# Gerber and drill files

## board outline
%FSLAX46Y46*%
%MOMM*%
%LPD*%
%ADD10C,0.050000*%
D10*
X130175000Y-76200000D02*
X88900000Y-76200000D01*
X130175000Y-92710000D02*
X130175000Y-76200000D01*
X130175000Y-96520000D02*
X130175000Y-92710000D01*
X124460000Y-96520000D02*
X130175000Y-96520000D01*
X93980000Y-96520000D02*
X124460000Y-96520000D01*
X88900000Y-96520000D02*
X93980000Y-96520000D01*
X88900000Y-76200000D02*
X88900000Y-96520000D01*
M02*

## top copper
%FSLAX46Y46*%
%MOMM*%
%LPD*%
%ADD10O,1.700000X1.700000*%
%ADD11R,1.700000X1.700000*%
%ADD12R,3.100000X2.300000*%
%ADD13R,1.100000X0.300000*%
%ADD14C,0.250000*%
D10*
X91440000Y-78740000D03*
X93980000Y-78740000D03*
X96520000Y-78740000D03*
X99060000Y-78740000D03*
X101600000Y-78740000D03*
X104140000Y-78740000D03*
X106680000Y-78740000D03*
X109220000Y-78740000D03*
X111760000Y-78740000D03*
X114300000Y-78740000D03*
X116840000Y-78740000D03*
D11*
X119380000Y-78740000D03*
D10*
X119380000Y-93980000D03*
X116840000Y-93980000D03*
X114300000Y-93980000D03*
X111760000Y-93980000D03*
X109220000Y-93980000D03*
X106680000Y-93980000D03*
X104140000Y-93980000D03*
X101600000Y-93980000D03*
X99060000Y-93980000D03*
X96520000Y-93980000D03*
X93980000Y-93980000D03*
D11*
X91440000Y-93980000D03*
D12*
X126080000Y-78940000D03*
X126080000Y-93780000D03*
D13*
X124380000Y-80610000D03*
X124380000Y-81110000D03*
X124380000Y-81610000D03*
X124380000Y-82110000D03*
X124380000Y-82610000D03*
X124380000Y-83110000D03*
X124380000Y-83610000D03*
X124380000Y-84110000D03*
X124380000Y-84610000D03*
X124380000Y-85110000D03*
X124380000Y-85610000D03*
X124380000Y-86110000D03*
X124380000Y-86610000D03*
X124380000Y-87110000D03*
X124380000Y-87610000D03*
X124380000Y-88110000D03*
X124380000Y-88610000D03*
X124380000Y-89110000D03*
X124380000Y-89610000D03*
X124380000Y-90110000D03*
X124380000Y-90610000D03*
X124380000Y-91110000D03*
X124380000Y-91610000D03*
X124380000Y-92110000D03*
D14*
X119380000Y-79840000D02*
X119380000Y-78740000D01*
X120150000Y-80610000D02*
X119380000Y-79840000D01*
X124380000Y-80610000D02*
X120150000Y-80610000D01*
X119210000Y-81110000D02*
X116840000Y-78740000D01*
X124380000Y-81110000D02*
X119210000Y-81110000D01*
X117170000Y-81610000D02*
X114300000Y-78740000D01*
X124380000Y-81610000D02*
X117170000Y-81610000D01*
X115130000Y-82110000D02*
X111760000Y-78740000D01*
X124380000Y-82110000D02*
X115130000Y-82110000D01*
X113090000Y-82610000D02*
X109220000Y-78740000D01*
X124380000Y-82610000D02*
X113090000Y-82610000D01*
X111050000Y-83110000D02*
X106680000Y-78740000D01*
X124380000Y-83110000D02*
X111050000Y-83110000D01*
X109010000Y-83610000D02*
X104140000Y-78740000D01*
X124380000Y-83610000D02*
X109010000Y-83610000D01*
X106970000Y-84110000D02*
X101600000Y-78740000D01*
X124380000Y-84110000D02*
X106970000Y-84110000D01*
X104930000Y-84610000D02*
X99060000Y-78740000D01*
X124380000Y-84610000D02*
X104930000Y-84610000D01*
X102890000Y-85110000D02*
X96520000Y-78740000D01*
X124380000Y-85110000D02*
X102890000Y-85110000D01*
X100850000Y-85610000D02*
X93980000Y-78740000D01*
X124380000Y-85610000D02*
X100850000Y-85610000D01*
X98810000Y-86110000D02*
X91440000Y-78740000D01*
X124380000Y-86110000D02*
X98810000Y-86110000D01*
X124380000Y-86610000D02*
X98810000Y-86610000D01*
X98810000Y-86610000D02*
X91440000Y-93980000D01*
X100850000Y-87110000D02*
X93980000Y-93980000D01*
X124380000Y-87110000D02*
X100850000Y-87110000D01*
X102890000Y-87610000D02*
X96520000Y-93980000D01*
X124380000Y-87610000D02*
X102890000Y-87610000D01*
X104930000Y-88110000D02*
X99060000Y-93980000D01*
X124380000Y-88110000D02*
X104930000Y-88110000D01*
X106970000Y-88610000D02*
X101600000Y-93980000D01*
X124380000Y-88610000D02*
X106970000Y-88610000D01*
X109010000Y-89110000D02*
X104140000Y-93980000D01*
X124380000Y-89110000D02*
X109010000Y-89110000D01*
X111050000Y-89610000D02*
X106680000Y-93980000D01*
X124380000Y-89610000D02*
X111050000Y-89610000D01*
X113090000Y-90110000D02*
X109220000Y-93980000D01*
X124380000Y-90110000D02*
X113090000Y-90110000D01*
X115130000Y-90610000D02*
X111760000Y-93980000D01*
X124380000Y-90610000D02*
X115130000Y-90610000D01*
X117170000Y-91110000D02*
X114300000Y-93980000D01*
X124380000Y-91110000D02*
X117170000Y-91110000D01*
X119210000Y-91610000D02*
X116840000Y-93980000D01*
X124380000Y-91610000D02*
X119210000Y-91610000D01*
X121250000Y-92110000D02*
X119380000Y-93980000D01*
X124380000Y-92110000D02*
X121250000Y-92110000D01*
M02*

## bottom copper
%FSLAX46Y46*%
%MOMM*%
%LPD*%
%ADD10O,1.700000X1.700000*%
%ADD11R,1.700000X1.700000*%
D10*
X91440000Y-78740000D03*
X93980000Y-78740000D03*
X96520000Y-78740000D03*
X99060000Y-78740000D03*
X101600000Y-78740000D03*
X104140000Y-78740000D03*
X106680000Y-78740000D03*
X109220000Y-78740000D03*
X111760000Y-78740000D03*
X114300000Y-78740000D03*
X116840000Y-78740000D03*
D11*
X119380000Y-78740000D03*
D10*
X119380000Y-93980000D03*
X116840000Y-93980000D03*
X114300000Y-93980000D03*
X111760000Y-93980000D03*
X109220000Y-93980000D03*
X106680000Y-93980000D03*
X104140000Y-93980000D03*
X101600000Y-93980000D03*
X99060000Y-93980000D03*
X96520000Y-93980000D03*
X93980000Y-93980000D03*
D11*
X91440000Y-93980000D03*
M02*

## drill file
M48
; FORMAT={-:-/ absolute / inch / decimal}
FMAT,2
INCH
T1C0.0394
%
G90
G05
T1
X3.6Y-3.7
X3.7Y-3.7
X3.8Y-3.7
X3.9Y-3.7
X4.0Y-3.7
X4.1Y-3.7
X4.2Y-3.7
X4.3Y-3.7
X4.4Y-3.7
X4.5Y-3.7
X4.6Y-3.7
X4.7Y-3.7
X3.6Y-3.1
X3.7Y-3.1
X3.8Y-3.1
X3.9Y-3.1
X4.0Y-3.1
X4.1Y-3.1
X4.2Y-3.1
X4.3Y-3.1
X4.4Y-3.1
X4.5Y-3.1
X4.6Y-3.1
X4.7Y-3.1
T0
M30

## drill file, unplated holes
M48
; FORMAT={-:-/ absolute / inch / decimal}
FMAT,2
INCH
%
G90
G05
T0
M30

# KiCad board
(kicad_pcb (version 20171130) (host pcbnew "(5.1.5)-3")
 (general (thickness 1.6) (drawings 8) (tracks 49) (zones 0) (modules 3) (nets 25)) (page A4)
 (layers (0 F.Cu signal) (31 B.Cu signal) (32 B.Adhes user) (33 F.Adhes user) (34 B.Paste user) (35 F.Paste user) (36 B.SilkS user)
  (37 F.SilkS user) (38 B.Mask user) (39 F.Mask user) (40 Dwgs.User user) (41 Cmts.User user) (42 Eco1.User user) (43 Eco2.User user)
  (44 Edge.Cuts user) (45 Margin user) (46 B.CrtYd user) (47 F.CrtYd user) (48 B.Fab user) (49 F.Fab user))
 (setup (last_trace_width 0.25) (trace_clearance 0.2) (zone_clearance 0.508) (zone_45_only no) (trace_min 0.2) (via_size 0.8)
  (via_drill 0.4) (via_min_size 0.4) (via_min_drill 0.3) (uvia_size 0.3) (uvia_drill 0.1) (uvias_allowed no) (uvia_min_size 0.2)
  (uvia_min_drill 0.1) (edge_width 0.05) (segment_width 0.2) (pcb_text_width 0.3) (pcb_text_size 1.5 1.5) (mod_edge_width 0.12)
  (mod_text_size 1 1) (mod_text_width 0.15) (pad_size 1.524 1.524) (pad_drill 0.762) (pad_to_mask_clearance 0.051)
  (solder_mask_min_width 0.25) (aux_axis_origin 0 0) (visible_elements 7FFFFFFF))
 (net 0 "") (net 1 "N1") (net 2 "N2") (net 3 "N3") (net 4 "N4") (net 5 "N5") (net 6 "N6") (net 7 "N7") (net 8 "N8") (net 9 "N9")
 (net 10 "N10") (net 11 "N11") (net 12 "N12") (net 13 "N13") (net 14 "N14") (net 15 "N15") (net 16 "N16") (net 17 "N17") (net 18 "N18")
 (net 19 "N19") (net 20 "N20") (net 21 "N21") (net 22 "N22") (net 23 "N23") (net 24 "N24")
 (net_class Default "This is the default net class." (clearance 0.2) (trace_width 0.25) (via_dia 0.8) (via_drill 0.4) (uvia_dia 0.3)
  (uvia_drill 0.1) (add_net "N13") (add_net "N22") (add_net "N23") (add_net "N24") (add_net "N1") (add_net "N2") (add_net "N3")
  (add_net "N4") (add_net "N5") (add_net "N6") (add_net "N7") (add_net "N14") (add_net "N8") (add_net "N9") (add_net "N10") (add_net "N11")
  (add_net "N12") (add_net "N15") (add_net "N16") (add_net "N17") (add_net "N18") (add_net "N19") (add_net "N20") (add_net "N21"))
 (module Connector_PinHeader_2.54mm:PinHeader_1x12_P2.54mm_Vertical (layer F.Cu) (at 119.38 78.74 270)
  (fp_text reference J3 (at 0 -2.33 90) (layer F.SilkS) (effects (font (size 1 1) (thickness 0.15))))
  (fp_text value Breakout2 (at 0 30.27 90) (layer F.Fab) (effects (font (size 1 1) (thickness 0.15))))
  (pad 12 thru_hole oval (at 0 27.94 270) (size 1.7 1.7) (drill 1) (layers *.Cu *.Mask) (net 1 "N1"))
  (pad 11 thru_hole oval (at 0 25.4 270) (size 1.7 1.7) (drill 1) (layers *.Cu *.Mask) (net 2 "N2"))
  (pad 10 thru_hole oval (at 0 22.86 270) (size 1.7 1.7) (drill 1) (layers *.Cu *.Mask) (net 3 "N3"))
  (pad 9 thru_hole oval (at 0 20.32 270) (size 1.7 1.7) (drill 1) (layers *.Cu *.Mask) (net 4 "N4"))
  (pad 8 thru_hole oval (at 0 17.78 270) (size 1.7 1.7) (drill 1) (layers *.Cu *.Mask) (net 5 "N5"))
  (pad 7 thru_hole oval (at 0 15.24 270) (size 1.7 1.7) (drill 1) (layers *.Cu *.Mask) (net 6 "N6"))
  (pad 6 thru_hole oval (at 0 12.7 270) (size 1.7 1.7) (drill 1) (layers *.Cu *.Mask) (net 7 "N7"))
  (pad 5 thru_hole oval (at 0 10.16 270) (size 1.7 1.7) (drill 1) (layers *.Cu *.Mask) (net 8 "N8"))
  (pad 4 thru_hole oval (at 0 7.62 270) (size 1.7 1.7) (drill 1) (layers *.Cu *.Mask) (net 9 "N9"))
  (pad 3 thru_hole oval (at 0 5.08 270) (size 1.7 1.7) (drill 1) (layers *.Cu *.Mask) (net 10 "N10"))
  (pad 2 thru_hole oval (at 0 2.54 270) (size 1.7 1.7) (drill 1) (layers *.Cu *.Mask) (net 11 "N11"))
  (pad 1 thru_hole rect (at 0 0 270) (size 1.7 1.7) (drill 1) (layers *.Cu *.Mask) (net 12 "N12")))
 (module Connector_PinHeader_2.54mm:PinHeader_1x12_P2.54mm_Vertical (layer F.Cu) (at 91.44 93.98 90)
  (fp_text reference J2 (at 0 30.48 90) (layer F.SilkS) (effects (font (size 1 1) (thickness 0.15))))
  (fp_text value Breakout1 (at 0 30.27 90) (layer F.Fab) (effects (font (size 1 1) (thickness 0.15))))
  (pad 12 thru_hole oval (at 0 27.94 90) (size 1.7 1.7) (drill 1) (layers *.Cu *.Mask) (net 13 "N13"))
  (pad 11 thru_hole oval (at 0 25.4 90) (size 1.7 1.7) (drill 1) (layers *.Cu *.Mask) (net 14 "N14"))
  (pad 10 thru_hole oval (at 0 22.86 90) (size 1.7 1.7) (drill 1) (layers *.Cu *.Mask) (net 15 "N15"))
  (pad 9 thru_hole oval (at 0 20.32 90) (size 1.7 1.7) (drill 1) (layers *.Cu *.Mask) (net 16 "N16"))
  (pad 8 thru_hole oval (at 0 17.78 90) (size 1.7 1.7) (drill 1) (layers *.Cu *.Mask) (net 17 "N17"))
  (pad 7 thru_hole oval (at 0 15.24 90) (size 1.7 1.7) (drill 1) (layers *.Cu *.Mask) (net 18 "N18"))
  (pad 6 thru_hole oval (at 0 12.7 90) (size 1.7 1.7) (drill 1) (layers *.Cu *.Mask) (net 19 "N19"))
  (pad 5 thru_hole oval (at 0 10.16 90) (size 1.7 1.7) (drill 1) (layers *.Cu *.Mask) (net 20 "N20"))
  (pad 4 thru_hole oval (at 0 7.62 90) (size 1.7 1.7) (drill 1) (layers *.Cu *.Mask) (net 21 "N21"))
  (pad 3 thru_hole oval (at 0 5.08 90) (size 1.7 1.7) (drill 1) (layers *.Cu *.Mask) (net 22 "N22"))
  (pad 2 thru_hole oval (at 0 2.54 90) (size 1.7 1.7) (drill 1) (layers *.Cu *.Mask) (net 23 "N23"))
  (pad 1 thru_hole rect (at 0 0 90) (size 1.7 1.7) (drill 1) (layers *.Cu *.Mask) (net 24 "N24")))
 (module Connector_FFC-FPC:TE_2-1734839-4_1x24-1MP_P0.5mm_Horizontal (layer F.Cu) (at 125.73 86.36 90)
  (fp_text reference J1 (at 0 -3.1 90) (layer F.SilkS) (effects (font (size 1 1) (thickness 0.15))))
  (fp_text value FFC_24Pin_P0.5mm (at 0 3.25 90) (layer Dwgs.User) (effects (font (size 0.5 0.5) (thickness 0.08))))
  (pad MP smd rect (at 7.42 0.35 90) (size 2.3 3.1) (layers F.Cu F.Paste F.Mask))
  (pad MP smd rect (at -7.42 0.35 90) (size 2.3 3.1) (layers F.Cu F.Paste F.Mask))
  (pad 24 smd rect (at 5.75 -1.35 90) (size 0.3 1.1) (layers F.Cu F.Paste F.Mask) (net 12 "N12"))
  (pad 23 smd rect (at 5.25 -1.35 90) (size 0.3 1.1) (layers F.Cu F.Paste F.Mask) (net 11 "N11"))
  (pad 22 smd rect (at 4.75 -1.35 90) (size 0.3 1.1) (layers F.Cu F.Paste F.Mask) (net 10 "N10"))
  (pad 21 smd rect (at 4.25 -1.35 90) (size 0.3 1.1) (layers F.Cu F.Paste F.Mask) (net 9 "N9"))
  (pad 20 smd rect (at 3.75 -1.35 90) (size 0.3 1.1) (layers F.Cu F.Paste F.Mask) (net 8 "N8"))
  (pad 19 smd rect (at 3.25 -1.35 90) (size 0.3 1.1) (layers F.Cu F.Paste F.Mask) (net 7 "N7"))
  (pad 18 smd rect (at 2.75 -1.35 90) (size 0.3 1.1) (layers F.Cu F.Paste F.Mask) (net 6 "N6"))
  (pad 17 smd rect (at 2.25 -1.35 90) (size 0.3 1.1) (layers F.Cu F.Paste F.Mask) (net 5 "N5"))
  (pad 16 smd rect (at 1.75 -1.35 90) (size 0.3 1.1) (layers F.Cu F.Paste F.Mask) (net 4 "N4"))
  (pad 15 smd rect (at 1.25 -1.35 90) (size 0.3 1.1) (layers F.Cu F.Paste F.Mask) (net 3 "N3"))
  (pad 14 smd rect (at 0.75 -1.35 90) (size 0.3 1.1) (layers F.Cu F.Paste F.Mask) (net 2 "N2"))
  (pad 13 smd rect (at 0.25 -1.35 90) (size 0.3 1.1) (layers F.Cu F.Paste F.Mask) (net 1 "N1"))
  (pad 12 smd rect (at -0.25 -1.35 90) (size 0.3 1.1) (layers F.Cu F.Paste F.Mask) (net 24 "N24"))
  (pad 11 smd rect (at -0.75 -1.35 90) (size 0.3 1.1) (layers F.Cu F.Paste F.Mask) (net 23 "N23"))
  (pad 10 smd rect (at -1.25 -1.35 90) (size 0.3 1.1) (layers F.Cu F.Paste F.Mask) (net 22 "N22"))
  (pad 9 smd rect (at -1.75 -1.35 90) (size 0.3 1.1) (layers F.Cu F.Paste F.Mask) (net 21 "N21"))
  (pad 8 smd rect (at -2.25 -1.35 90) (size 0.3 1.1) (layers F.Cu F.Paste F.Mask) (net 20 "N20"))
  (pad 7 smd rect (at -2.75 -1.35 90) (size 0.3 1.1) (layers F.Cu F.Paste F.Mask) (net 19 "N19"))
  (pad 6 smd rect (at -3.25 -1.35 90) (size 0.3 1.1) (layers F.Cu F.Paste F.Mask) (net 18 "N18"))
  (pad 5 smd rect (at -3.75 -1.35 90) (size 0.3 1.1) (layers F.Cu F.Paste F.Mask) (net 17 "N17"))
  (pad 4 smd rect (at -4.25 -1.35 90) (size 0.3 1.1) (layers F.Cu F.Paste F.Mask) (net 16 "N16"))
  (pad 3 smd rect (at -4.75 -1.35 90) (size 0.3 1.1) (layers F.Cu F.Paste F.Mask) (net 15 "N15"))
  (pad 2 smd rect (at -5.25 -1.35 90) (size 0.3 1.1) (layers F.Cu F.Paste F.Mask) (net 14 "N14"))
  (pad 1 smd rect (at -5.75 -1.35 90) (size 0.3 1.1) (layers F.Cu F.Paste F.Mask) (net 13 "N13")))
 (gr_line (start 130.175 76.2) (end 88.9 76.2) (layer Edge.Cuts) (width 0.05))
 (gr_line (start 130.175 92.71) (end 130.175 76.2) (layer Edge.Cuts) (width 0.05))
 (gr_line (start 130.175 96.52) (end 130.175 92.71) (layer Edge.Cuts) (width 0.05))
 (gr_line (start 124.46 96.52) (end 130.175 96.52) (layer Edge.Cuts) (width 0.05))
 (gr_line (start 93.98 96.52) (end 124.46 96.52) (layer Edge.Cuts) (width 0.05))
 (gr_line (start 88.9 96.52) (end 93.98 96.52) (layer Edge.Cuts) (width 0.05))
 (gr_line (start 88.9 76.2) (end 88.9 96.52) (layer Edge.Cuts) (width 0.05))
 (segment (start 119.38 79.84) (end 119.38 78.74) (width 0.25) (layer F.Cu) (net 12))
 (segment (start 120.15 80.61) (end 119.38 79.84) (width 0.25) (layer F.Cu) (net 12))
 (segment (start 124.38 80.61) (end 120.15 80.61) (width 0.25) (layer F.Cu) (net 12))
 (segment (start 119.21 81.11) (end 116.84 78.74) (width 0.25) (layer F.Cu) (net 11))
 (segment (start 124.38 81.11) (end 119.21 81.11) (width 0.25) (layer F.Cu) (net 11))
 (segment (start 117.17 81.61) (end 114.3 78.74) (width 0.25) (layer F.Cu) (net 10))
 (segment (start 124.38 81.61) (end 117.17 81.61) (width 0.25) (layer F.Cu) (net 10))
 (segment (start 115.13 82.11) (end 111.76 78.74) (width 0.25) (layer F.Cu) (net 9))
 (segment (start 124.38 82.11) (end 115.13 82.11) (width 0.25) (layer F.Cu) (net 9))
 (segment (start 113.09 82.61) (end 109.22 78.74) (width 0.25) (layer F.Cu) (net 8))
 (segment (start 124.38 82.61) (end 113.09 82.61) (width 0.25) (layer F.Cu) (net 8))
 (segment (start 111.05 83.11) (end 106.68 78.74) (width 0.25) (layer F.Cu) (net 7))
 (segment (start 124.38 83.11) (end 111.05 83.11) (width 0.25) (layer F.Cu) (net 7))
 (segment (start 109.01 83.61) (end 104.14 78.74) (width 0.25) (layer F.Cu) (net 6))
 (segment (start 124.38 83.61) (end 109.01 83.61) (width 0.25) (layer F.Cu) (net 6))
 (segment (start 106.97 84.11) (end 101.6 78.74) (width 0.25) (layer F.Cu) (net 5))
 (segment (start 124.38 84.11) (end 106.97 84.11) (width 0.25) (layer F.Cu) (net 5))
 (segment (start 104.93 84.61) (end 99.06 78.74) (width 0.25) (layer F.Cu) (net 4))
 (segment (start 124.38 84.61) (end 104.93 84.61) (width 0.25) (layer F.Cu) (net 4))
 (segment (start 102.89 85.11) (end 96.52 78.74) (width 0.25) (layer F.Cu) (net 3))
 (segment (start 124.38 85.11) (end 102.89 85.11) (width 0.25) (layer F.Cu) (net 3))
 (segment (start 100.85 85.61) (end 93.98 78.74) (width 0.25) (layer F.Cu) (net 2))
 (segment (start 124.38 85.61) (end 100.85 85.61) (width 0.25) (layer F.Cu) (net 2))
 (segment (start 98.81 86.11) (end 91.44 78.74) (width 0.25) (layer F.Cu) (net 1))
 (segment (start 124.38 86.11) (end 98.81 86.11) (width 0.25) (layer F.Cu) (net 1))
 (segment (start 124.38 86.61) (end 98.81 86.61) (width 0.25) (layer F.Cu) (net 24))
 (segment (start 98.81 86.61) (end 91.44 93.98) (width 0.25) (layer F.Cu) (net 24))
 (segment (start 100.85 87.11) (end 93.98 93.98) (width 0.25) (layer F.Cu) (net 23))
 (segment (start 124.38 87.11) (end 100.85 87.11) (width 0.25) (layer F.Cu) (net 23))
 (segment (start 102.89 87.61) (end 96.52 93.98) (width 0.25) (layer F.Cu) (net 22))
 (segment (start 124.38 87.61) (end 102.89 87.61) (width 0.25) (layer F.Cu) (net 22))
 (segment (start 104.93 88.11) (end 99.06 93.98) (width 0.25) (layer F.Cu) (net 21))
 (segment (start 124.38 88.11) (end 104.93 88.11) (width 0.25) (layer F.Cu) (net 21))
 (segment (start 106.97 88.61) (end 101.6 93.98) (width 0.25) (layer F.Cu) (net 20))
 (segment (start 124.38 88.61) (end 106.97 88.61) (width 0.25) (layer F.Cu) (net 20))
 (segment (start 109.01 89.11) (end 104.14 93.98) (width 0.25) (layer F.Cu) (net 19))
 (segment (start 124.38 89.11) (end 109.01 89.11) (width 0.25) (layer F.Cu) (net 19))
 (segment (start 111.05 89.61) (end 106.68 93.98) (width 0.25) (layer F.Cu) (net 18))
 (segment (start 124.38 89.61) (end 111.05 89.61) (width 0.25) (layer F.Cu) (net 18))
 (segment (start 113.09 90.11) (end 109.22 93.98) (width 0.25) (layer F.Cu) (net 17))
 (segment (start 124.38 90.11) (end 113.09 90.11) (width 0.25) (layer F.Cu) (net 17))
 (segment (start 115.13 90.61) (end 111.76 93.98) (width 0.25) (layer F.Cu) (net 16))
 (segment (start 124.38 90.61) (end 115.13 90.61) (width 0.25) (layer F.Cu) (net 16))
 (segment (start 117.17 91.11) (end 114.3 93.98) (width 0.25) (layer F.Cu) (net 15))
 (segment (start 124.38 91.11) (end 117.17 91.11) (width 0.25) (layer F.Cu) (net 15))
 (segment (start 119.21 91.61) (end 116.84 93.98) (width 0.25) (layer F.Cu) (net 14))
 (segment (start 124.38 91.61) (end 119.21 91.61) (width 0.25) (layer F.Cu) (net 14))
 (segment (start 121.25 92.11) (end 119.38 93.98) (width 0.25) (layer F.Cu) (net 13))
 (segment (start 124.38 92.11) (end 121.25 92.11) (width 0.25) (layer F.Cu) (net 13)))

